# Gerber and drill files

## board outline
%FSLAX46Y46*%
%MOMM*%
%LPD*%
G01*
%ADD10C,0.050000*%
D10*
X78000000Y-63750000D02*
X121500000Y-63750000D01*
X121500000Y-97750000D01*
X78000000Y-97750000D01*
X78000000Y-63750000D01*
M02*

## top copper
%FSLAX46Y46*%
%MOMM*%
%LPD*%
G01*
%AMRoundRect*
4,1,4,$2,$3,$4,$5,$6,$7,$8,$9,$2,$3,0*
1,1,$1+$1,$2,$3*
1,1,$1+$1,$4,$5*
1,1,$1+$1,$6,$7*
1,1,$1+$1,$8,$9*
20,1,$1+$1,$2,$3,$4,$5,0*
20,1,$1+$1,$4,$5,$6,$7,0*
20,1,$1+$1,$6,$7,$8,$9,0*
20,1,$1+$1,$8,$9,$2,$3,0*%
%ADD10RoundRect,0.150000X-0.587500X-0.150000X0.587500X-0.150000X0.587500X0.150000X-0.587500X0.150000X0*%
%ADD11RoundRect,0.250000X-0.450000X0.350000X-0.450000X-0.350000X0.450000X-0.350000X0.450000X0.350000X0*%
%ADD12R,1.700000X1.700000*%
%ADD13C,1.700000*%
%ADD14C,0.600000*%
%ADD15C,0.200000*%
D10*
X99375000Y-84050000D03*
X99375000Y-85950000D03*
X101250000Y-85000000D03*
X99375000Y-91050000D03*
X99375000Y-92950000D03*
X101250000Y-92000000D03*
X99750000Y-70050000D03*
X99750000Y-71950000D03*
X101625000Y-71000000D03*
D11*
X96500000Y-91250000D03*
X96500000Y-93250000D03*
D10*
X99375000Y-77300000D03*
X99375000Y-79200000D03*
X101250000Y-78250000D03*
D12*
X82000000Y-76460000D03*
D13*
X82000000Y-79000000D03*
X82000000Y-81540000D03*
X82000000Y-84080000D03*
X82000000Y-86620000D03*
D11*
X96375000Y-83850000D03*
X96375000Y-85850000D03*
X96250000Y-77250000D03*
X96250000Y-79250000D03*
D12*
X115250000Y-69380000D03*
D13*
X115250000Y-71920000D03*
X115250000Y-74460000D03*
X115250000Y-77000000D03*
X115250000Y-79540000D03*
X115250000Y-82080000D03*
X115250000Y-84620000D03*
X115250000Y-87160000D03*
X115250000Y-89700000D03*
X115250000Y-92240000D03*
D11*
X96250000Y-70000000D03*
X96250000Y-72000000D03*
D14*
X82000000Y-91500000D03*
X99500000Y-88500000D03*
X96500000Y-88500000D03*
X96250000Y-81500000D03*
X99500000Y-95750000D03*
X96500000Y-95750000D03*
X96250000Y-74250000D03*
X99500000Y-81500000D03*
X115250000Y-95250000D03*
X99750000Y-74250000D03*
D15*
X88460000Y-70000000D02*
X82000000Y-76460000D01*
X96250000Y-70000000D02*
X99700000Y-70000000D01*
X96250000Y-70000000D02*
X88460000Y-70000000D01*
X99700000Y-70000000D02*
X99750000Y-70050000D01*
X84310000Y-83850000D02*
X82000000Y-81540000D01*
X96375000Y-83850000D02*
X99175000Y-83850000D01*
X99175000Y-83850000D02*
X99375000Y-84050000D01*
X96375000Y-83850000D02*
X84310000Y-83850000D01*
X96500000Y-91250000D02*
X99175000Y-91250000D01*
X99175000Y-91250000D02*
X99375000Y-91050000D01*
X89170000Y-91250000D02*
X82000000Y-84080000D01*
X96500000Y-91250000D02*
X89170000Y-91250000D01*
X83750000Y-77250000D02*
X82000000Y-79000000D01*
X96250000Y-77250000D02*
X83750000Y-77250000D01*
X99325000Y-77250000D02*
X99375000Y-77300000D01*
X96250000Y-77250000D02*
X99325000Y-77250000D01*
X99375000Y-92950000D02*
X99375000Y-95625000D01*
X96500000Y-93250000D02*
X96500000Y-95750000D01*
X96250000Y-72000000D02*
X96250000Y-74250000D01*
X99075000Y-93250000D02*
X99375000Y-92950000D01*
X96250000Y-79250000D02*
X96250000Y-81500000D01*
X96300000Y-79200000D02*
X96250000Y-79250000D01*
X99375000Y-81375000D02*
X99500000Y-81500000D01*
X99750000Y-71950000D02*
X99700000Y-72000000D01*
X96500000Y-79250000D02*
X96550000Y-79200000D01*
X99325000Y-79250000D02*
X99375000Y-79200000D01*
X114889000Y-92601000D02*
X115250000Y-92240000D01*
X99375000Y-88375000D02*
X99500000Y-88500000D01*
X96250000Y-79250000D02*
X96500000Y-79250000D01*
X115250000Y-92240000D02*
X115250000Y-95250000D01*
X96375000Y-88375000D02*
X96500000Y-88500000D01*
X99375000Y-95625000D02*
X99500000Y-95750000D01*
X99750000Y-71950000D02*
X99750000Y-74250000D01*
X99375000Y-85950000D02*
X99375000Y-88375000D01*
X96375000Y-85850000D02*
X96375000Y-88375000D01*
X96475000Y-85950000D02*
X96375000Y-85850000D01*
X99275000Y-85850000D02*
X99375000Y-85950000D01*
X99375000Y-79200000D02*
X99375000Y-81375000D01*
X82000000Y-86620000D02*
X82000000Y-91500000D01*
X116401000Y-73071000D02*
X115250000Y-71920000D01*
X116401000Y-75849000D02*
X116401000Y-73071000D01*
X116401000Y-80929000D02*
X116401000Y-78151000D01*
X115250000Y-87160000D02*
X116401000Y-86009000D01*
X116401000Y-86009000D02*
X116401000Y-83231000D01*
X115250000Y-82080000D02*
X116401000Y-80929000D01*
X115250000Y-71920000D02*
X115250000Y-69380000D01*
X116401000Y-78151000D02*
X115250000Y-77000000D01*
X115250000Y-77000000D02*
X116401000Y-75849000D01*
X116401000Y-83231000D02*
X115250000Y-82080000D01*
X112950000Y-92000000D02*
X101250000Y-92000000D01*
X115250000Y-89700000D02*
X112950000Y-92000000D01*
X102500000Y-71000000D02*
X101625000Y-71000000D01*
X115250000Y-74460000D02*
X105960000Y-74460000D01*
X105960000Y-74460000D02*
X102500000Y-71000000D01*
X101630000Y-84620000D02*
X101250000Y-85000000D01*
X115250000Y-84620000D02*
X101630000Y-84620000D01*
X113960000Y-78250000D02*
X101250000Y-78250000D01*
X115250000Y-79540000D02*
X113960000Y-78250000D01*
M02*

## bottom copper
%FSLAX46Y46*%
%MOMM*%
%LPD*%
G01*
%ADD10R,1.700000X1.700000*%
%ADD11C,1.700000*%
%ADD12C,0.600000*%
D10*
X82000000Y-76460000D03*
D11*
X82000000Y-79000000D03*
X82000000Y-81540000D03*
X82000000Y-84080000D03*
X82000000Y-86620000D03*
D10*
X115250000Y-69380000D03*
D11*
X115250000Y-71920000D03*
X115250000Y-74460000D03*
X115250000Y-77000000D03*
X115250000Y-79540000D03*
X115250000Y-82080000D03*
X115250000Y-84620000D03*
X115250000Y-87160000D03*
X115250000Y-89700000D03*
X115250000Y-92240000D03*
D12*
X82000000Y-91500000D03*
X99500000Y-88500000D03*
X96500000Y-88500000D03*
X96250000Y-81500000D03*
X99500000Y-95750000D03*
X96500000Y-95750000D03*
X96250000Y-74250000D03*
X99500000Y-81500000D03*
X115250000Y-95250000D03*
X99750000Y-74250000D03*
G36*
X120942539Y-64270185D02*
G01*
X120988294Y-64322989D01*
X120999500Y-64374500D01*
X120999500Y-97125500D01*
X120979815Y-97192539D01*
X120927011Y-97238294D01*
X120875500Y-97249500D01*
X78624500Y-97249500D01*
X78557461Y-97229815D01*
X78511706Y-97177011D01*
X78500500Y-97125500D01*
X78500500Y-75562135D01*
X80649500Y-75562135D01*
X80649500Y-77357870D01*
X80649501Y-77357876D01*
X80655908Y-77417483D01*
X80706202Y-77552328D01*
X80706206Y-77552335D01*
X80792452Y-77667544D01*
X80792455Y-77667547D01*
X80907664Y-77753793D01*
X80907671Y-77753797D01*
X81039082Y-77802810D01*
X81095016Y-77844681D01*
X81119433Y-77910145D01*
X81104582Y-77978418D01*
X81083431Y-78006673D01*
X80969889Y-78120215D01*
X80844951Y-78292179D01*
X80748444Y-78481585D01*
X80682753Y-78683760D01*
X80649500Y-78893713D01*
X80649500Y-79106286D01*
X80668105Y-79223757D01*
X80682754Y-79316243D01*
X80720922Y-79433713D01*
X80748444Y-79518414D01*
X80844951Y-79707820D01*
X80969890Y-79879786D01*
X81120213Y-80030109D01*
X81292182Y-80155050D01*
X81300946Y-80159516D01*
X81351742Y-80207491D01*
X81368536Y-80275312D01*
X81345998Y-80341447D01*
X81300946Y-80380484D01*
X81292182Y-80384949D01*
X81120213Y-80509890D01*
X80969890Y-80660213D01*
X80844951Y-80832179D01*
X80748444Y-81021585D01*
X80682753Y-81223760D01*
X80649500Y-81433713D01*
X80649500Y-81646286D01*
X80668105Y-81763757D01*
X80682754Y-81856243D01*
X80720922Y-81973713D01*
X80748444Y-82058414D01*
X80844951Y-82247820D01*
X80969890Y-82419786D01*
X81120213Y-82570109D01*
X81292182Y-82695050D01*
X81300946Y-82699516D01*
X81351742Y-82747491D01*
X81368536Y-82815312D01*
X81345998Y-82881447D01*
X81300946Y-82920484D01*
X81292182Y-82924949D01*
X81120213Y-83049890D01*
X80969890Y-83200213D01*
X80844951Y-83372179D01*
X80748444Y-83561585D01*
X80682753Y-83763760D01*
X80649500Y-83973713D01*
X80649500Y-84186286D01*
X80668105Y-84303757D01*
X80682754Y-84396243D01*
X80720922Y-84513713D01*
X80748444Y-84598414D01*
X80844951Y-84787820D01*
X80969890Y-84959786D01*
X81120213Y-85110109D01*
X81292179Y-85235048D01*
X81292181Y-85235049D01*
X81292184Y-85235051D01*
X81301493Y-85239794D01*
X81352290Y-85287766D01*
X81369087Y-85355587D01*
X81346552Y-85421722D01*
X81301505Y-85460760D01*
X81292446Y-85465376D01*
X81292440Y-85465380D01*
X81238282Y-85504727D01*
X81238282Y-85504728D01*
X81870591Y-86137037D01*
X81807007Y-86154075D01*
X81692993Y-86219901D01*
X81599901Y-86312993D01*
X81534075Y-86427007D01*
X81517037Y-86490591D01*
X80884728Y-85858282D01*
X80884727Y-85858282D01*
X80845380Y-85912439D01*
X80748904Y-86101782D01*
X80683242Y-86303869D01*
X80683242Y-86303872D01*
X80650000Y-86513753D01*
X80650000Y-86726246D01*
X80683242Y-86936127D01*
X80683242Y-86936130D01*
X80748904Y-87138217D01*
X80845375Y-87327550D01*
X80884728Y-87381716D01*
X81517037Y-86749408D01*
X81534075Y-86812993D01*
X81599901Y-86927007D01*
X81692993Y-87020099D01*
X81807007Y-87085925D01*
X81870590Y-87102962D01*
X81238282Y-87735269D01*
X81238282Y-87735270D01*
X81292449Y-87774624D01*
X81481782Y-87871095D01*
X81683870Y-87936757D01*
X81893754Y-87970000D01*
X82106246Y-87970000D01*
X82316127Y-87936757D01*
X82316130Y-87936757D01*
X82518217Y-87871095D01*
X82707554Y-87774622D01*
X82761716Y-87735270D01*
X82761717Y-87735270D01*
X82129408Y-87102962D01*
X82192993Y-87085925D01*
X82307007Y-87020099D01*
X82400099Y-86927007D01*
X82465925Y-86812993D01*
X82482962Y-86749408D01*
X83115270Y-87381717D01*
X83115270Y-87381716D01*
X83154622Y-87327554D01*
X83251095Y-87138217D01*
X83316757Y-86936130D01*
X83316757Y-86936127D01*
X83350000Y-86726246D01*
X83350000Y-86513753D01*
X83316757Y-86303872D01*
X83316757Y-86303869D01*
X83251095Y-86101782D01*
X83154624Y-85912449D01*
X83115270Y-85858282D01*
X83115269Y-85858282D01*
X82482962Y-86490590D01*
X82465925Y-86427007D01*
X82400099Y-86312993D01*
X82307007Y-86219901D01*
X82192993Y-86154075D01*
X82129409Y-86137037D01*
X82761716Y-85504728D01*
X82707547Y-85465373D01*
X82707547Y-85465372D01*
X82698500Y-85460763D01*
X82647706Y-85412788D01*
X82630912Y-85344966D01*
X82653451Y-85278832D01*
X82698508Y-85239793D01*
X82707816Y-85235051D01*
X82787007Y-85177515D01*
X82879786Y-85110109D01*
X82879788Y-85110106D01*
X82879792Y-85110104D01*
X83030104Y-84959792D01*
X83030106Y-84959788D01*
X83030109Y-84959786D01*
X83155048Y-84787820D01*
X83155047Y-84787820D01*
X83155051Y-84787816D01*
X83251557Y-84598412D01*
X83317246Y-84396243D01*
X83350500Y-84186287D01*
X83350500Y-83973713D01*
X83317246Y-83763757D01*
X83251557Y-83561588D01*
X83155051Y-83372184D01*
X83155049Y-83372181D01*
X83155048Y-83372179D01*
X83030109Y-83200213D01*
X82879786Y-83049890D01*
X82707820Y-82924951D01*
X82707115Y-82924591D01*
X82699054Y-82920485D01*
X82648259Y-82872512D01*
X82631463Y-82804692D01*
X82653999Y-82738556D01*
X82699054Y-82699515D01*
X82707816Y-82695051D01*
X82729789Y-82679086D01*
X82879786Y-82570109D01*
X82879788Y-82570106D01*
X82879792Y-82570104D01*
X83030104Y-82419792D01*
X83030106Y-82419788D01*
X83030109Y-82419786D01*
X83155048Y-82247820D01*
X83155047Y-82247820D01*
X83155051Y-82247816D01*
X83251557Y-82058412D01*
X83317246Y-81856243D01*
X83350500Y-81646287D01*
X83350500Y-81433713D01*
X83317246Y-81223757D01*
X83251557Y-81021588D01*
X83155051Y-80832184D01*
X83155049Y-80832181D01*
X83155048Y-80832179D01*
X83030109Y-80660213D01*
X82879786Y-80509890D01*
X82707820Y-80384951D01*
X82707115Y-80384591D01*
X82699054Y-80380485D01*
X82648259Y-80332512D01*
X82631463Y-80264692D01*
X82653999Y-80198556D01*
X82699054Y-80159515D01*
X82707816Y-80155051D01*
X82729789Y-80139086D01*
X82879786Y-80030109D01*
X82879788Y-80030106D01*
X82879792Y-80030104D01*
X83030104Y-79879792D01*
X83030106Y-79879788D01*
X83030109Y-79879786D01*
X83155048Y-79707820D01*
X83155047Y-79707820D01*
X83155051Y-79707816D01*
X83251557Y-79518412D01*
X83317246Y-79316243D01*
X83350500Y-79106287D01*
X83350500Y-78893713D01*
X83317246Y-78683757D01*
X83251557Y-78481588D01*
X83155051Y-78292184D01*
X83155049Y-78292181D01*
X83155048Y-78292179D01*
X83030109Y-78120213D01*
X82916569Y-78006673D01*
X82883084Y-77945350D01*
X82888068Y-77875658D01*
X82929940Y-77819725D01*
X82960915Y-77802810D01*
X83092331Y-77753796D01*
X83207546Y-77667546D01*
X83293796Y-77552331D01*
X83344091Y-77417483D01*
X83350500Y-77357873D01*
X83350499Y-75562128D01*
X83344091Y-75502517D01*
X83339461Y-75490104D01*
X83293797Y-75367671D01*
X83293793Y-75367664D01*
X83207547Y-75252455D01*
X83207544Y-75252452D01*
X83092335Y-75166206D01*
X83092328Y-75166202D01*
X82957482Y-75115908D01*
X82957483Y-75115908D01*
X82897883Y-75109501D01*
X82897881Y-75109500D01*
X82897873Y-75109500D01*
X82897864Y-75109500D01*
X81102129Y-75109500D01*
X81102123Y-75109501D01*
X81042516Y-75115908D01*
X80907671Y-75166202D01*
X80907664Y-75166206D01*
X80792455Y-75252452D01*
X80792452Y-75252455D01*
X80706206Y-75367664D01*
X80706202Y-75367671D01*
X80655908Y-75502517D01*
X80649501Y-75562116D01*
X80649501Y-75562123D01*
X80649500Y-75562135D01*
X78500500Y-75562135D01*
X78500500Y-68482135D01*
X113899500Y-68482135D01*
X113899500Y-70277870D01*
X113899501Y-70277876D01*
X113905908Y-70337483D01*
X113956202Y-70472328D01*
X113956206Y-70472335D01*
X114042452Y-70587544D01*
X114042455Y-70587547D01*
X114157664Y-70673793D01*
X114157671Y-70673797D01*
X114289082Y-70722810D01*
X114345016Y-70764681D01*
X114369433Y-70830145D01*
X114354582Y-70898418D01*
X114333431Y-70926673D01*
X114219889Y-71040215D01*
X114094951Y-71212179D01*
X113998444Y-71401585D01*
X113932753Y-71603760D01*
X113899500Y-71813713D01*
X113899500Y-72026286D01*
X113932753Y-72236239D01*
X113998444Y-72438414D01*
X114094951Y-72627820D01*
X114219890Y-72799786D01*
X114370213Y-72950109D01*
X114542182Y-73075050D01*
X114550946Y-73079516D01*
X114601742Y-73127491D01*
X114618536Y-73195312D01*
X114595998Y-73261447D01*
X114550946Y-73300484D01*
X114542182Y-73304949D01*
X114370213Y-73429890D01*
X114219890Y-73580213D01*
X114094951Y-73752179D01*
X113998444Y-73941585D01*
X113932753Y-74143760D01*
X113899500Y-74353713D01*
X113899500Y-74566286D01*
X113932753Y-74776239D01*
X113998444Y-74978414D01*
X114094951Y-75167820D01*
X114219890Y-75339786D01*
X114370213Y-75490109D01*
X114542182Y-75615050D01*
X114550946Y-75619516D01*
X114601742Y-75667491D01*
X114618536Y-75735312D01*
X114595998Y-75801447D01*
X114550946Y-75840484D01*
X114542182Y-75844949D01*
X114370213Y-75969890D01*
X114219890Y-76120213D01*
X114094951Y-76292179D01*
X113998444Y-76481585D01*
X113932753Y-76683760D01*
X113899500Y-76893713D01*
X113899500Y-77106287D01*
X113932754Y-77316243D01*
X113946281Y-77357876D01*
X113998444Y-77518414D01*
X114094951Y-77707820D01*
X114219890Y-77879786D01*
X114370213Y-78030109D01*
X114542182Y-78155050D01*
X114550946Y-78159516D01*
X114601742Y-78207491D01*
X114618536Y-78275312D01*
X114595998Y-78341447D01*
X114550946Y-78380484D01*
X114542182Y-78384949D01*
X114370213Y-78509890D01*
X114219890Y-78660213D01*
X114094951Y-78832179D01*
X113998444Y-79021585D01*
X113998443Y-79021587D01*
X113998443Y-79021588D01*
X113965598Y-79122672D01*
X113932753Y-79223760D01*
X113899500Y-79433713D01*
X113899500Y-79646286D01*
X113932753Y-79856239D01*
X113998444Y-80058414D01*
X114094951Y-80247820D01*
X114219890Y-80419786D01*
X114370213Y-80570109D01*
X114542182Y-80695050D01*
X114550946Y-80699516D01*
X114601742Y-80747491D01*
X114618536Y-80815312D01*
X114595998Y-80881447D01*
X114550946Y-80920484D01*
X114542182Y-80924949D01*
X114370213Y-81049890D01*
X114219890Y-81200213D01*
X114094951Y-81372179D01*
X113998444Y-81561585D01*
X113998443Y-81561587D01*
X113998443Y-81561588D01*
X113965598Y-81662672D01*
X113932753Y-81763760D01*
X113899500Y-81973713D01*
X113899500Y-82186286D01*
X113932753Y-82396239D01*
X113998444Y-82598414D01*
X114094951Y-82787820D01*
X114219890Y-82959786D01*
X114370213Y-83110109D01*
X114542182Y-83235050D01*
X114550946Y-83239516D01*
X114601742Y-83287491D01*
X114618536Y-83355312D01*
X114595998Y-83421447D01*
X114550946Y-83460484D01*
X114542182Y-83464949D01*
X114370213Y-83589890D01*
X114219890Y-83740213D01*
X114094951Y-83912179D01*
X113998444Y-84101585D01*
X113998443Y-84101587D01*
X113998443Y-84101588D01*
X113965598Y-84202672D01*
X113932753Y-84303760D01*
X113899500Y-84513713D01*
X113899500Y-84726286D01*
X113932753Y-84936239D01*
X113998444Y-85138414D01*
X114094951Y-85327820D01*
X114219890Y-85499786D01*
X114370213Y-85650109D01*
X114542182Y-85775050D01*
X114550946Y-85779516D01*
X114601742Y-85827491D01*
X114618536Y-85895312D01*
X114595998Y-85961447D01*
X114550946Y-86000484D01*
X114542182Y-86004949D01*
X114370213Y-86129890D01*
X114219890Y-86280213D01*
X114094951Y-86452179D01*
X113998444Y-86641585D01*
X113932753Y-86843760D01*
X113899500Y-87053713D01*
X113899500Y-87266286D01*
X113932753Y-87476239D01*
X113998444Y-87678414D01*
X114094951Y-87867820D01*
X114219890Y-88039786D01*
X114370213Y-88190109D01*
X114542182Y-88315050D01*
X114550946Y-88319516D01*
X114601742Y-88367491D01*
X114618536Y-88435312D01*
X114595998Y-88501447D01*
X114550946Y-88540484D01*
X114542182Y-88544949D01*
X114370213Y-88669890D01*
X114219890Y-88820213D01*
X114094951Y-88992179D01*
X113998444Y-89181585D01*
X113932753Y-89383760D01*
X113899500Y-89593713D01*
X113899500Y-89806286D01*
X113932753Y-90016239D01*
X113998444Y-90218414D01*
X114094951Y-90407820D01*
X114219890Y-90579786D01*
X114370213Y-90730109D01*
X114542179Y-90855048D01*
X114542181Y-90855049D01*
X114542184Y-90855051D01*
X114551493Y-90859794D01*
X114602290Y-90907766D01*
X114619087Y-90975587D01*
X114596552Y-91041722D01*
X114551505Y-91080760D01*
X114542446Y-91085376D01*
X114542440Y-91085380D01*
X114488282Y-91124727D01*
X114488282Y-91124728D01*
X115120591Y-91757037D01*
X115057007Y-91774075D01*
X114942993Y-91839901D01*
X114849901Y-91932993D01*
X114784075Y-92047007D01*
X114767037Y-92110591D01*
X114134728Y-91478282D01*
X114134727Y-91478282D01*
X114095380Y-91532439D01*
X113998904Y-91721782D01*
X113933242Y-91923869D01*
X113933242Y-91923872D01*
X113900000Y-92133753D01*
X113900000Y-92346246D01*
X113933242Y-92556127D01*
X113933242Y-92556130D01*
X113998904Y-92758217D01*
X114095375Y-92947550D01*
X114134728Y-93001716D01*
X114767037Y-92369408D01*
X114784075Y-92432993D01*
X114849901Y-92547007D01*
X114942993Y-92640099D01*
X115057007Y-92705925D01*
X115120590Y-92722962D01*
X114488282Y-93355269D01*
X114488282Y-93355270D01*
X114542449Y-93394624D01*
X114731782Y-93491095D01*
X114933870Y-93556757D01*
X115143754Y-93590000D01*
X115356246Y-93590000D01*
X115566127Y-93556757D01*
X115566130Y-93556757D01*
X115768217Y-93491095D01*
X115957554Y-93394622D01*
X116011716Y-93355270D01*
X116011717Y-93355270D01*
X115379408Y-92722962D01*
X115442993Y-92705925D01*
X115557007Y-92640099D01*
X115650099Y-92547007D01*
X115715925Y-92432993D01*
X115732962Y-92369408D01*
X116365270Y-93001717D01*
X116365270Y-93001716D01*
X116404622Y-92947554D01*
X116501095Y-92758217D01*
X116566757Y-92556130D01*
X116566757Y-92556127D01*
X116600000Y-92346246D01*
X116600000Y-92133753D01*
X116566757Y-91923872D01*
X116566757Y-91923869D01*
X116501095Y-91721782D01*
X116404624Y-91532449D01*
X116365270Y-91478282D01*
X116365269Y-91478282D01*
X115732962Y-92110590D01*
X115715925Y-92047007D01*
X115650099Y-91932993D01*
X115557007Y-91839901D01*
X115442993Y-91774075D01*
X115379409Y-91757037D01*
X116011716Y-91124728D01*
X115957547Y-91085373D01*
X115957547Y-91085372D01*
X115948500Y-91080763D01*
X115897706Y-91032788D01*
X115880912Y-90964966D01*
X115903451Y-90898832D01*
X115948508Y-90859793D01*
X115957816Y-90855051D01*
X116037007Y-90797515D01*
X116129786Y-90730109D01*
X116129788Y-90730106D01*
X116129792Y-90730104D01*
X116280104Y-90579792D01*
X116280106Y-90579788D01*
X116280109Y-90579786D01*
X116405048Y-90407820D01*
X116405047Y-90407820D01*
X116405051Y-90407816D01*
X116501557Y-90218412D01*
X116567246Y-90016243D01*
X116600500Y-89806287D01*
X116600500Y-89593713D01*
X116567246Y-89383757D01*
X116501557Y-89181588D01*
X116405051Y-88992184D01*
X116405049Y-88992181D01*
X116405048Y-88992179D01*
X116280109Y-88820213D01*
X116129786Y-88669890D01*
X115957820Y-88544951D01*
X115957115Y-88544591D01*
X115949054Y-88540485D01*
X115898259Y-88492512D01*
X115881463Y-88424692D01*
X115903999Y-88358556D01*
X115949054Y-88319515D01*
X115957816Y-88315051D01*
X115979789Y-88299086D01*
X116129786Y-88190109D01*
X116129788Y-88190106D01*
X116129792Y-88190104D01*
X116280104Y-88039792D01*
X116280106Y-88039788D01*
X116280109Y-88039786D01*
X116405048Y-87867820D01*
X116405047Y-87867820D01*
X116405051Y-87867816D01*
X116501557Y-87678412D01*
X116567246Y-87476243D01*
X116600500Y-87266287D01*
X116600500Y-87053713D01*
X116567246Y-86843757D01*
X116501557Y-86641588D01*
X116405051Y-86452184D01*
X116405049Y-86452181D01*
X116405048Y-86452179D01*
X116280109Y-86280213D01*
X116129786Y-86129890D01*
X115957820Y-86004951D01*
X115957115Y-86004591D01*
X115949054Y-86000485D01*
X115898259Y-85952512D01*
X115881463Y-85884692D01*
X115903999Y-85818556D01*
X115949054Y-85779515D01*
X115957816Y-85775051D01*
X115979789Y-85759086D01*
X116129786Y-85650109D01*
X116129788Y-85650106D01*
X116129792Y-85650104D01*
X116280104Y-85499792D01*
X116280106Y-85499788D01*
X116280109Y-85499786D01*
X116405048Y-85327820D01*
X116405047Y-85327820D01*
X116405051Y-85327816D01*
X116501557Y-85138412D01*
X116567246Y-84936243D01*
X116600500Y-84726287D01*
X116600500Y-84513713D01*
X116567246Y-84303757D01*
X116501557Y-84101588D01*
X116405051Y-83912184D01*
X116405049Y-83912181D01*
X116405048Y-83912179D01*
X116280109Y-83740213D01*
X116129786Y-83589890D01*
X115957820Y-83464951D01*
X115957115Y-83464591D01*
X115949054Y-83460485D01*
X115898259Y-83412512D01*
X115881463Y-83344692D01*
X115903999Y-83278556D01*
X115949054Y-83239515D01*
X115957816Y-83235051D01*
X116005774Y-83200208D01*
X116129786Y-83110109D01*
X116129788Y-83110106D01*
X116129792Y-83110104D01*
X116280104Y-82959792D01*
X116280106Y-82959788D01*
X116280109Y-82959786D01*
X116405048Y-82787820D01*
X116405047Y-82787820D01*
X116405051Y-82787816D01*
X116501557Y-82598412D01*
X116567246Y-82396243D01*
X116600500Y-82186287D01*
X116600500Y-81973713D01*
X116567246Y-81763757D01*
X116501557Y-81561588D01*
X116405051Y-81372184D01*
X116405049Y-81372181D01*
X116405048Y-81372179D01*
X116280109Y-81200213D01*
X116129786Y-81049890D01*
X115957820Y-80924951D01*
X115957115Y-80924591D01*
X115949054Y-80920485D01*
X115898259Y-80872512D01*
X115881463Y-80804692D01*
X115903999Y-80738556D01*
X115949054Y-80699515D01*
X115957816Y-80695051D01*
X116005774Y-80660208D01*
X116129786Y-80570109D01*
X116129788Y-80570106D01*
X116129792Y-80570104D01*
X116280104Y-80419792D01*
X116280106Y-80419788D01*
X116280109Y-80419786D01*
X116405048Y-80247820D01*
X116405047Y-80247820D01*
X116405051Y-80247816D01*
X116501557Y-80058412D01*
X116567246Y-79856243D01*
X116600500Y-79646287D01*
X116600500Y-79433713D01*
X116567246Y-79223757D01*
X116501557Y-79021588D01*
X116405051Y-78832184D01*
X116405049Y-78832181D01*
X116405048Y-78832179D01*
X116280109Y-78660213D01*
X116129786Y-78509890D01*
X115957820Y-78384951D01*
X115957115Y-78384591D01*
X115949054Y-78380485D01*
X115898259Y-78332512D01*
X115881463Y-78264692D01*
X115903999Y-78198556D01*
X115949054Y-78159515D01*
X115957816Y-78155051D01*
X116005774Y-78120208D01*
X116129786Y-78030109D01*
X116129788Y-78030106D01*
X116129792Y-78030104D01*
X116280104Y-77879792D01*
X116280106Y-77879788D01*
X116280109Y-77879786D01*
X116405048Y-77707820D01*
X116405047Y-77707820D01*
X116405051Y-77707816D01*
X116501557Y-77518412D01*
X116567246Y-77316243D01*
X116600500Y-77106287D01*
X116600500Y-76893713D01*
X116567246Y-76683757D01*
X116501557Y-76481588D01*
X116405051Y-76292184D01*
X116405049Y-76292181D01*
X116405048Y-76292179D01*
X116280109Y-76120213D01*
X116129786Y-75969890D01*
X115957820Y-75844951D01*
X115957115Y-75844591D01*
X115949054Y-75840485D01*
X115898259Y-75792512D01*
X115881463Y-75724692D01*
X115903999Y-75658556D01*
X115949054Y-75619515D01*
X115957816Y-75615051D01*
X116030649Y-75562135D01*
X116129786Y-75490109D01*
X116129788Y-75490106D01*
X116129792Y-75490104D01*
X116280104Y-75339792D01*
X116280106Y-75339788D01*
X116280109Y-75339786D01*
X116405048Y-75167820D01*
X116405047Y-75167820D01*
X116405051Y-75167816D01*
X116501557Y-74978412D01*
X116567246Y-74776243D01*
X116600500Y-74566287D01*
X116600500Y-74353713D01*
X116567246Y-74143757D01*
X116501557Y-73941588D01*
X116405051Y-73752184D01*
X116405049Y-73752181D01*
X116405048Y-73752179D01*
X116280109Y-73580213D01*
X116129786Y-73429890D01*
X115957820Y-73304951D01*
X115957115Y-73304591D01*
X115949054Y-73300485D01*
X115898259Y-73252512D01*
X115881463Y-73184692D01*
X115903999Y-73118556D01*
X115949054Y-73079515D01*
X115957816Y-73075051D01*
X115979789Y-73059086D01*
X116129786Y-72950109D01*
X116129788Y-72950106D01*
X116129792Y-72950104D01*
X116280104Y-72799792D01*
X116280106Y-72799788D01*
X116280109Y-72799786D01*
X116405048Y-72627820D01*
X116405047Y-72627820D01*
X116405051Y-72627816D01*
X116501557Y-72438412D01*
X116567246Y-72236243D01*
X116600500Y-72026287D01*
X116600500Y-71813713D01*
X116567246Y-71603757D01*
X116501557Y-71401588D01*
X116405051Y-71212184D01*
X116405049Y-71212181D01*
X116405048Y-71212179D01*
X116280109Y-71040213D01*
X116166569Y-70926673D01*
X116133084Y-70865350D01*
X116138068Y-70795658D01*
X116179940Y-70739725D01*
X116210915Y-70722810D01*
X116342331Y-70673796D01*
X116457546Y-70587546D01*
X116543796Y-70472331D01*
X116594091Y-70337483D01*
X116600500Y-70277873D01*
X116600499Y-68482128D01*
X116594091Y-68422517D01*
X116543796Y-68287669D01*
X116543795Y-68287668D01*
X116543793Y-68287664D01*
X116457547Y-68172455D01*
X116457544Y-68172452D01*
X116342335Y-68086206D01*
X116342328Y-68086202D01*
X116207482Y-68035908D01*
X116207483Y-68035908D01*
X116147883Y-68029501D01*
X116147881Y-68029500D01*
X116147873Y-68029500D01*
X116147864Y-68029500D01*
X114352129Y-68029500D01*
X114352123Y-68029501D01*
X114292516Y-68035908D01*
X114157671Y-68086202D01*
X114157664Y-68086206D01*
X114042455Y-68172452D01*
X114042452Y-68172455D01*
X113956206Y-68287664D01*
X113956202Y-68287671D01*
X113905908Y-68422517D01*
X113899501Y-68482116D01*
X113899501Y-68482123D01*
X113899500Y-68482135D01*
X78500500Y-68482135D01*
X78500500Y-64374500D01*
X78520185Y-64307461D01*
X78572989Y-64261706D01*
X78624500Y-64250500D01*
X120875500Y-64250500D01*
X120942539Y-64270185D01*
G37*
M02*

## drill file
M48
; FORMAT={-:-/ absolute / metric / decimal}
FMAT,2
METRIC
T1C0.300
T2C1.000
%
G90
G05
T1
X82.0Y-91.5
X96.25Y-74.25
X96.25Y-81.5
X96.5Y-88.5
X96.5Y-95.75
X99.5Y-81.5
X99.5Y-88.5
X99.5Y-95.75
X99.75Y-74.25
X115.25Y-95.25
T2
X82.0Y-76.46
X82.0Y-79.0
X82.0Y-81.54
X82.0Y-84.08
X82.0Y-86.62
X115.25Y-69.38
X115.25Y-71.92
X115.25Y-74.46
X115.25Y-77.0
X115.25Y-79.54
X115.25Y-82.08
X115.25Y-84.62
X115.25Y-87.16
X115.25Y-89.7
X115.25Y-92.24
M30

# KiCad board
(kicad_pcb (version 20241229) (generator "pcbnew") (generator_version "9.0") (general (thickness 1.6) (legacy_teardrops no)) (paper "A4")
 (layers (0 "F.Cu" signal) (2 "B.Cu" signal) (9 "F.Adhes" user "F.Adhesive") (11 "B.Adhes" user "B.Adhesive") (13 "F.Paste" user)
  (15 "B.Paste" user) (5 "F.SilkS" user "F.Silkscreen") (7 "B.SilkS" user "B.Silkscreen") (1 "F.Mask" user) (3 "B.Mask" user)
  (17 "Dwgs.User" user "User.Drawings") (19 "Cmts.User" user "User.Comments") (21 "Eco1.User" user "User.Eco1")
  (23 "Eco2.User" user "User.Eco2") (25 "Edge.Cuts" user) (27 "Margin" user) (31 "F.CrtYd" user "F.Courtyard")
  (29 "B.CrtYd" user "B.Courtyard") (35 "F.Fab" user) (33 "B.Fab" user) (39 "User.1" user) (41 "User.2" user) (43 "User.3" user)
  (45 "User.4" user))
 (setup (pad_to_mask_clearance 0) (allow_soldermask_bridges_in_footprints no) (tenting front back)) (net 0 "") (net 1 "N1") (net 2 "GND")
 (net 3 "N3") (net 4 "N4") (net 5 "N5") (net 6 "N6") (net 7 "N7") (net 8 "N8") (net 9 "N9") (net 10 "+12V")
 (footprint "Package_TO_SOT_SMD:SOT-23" (layer "F.Cu") (at 100.3125 85)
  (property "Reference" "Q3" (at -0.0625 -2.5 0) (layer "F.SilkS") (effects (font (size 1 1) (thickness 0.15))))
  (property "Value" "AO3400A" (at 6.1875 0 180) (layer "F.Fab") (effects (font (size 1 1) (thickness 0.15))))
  (pad "1" smd roundrect (at -0.9375 -0.95) (size 1.475 0.6) (layers "F.Cu" "F.Mask" "F.Paste") (roundrect_rratio 0.25) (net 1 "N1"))
  (pad "2" smd roundrect (at -0.9375 0.95) (size 1.475 0.6) (layers "F.Cu" "F.Mask" "F.Paste") (roundrect_rratio 0.25) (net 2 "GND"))
  (pad "3" smd roundrect (at 0.9375 0) (size 1.475 0.6) (layers "F.Cu" "F.Mask" "F.Paste") (roundrect_rratio 0.25) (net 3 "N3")))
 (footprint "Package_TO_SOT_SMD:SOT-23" (layer "F.Cu") (at 100.3125 92)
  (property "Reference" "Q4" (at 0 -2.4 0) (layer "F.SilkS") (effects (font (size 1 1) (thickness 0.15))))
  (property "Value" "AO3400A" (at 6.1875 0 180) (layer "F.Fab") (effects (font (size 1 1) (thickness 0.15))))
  (pad "1" smd roundrect (at -0.9375 -0.95) (size 1.475 0.6) (layers "F.Cu" "F.Mask" "F.Paste") (roundrect_rratio 0.25) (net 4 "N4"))
  (pad "2" smd roundrect (at -0.9375 0.95) (size 1.475 0.6) (layers "F.Cu" "F.Mask" "F.Paste") (roundrect_rratio 0.25) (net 2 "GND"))
  (pad "3" smd roundrect (at 0.9375 0) (size 1.475 0.6) (layers "F.Cu" "F.Mask" "F.Paste") (roundrect_rratio 0.25) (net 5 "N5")))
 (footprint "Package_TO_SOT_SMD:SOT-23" (layer "F.Cu") (at 100.6875 71)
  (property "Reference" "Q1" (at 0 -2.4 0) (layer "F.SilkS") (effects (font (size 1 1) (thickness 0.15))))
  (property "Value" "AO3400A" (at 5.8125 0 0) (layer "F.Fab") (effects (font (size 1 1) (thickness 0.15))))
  (pad "1" smd roundrect (at -0.9375 -0.95) (size 1.475 0.6) (layers "F.Cu" "F.Mask" "F.Paste") (roundrect_rratio 0.25) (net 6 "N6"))
  (pad "2" smd roundrect (at -0.9375 0.95) (size 1.475 0.6) (layers "F.Cu" "F.Mask" "F.Paste") (roundrect_rratio 0.25) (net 2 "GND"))
  (pad "3" smd roundrect (at 0.9375 0) (size 1.475 0.6) (layers "F.Cu" "F.Mask" "F.Paste") (roundrect_rratio 0.25) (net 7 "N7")))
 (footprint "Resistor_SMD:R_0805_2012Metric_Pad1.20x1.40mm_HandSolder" (layer "F.Cu") (at 96.5 92.25 -90)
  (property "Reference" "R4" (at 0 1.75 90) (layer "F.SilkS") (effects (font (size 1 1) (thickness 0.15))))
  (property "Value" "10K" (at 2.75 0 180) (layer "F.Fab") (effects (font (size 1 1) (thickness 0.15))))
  (pad "1" smd roundrect (at -1 0 270) (size 1.2 1.4) (layers "F.Cu" "F.Mask" "F.Paste") (roundrect_rratio 0.208333) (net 4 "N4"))
  (pad "2" smd roundrect (at 1 0 270) (size 1.2 1.4) (layers "F.Cu" "F.Mask" "F.Paste") (roundrect_rratio 0.208333) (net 2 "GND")))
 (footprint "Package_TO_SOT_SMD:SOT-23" (layer "F.Cu") (at 100.3125 78.25)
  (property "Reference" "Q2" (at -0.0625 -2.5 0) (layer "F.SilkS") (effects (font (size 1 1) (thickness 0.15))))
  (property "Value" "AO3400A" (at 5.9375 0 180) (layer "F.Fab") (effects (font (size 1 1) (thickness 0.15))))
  (pad "1" smd roundrect (at -0.9375 -0.95) (size 1.475 0.6) (layers "F.Cu" "F.Mask" "F.Paste") (roundrect_rratio 0.25) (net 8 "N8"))
  (pad "2" smd roundrect (at -0.9375 0.95) (size 1.475 0.6) (layers "F.Cu" "F.Mask" "F.Paste") (roundrect_rratio 0.25) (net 2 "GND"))
  (pad "3" smd roundrect (at 0.9375 0) (size 1.475 0.6) (layers "F.Cu" "F.Mask" "F.Paste") (roundrect_rratio 0.25) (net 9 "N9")))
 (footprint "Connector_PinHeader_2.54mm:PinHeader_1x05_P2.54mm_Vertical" (layer "F.Cu") (at 82 76.46)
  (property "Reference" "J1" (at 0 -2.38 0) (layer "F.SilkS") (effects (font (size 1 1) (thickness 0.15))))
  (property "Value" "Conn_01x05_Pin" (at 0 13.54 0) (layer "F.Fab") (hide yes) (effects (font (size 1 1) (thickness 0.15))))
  (pad "1" thru_hole rect (at 0 0) (size 1.7 1.7) (drill 1) (layers "*.Cu" "*.Mask") (remove_unused_layers no) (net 6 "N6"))
  (pad "2" thru_hole circle (at 0 2.54) (size 1.7 1.7) (drill 1) (layers "*.Cu" "*.Mask") (remove_unused_layers no) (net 8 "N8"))
  (pad "3" thru_hole circle (at 0 5.08) (size 1.7 1.7) (drill 1) (layers "*.Cu" "*.Mask") (remove_unused_layers no) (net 1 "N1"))
  (pad "4" thru_hole circle (at 0 7.62) (size 1.7 1.7) (drill 1) (layers "*.Cu" "*.Mask") (remove_unused_layers no) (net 4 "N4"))
  (pad "5" thru_hole circle (at 0 10.16) (size 1.7 1.7) (drill 1) (layers "*.Cu" "*.Mask") (remove_unused_layers no) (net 2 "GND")))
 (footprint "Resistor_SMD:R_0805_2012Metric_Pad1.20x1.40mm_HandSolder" (layer "F.Cu") (at 96.375 84.85 -90)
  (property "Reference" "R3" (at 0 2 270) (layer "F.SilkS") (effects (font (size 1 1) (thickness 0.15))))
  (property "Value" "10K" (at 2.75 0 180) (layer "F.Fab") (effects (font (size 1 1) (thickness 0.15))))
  (pad "1" smd roundrect (at -1 0 270) (size 1.2 1.4) (layers "F.Cu" "F.Mask" "F.Paste") (roundrect_rratio 0.208333) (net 1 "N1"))
  (pad "2" smd roundrect (at 1 0 270) (size 1.2 1.4) (layers "F.Cu" "F.Mask" "F.Paste") (roundrect_rratio 0.208333) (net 2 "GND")))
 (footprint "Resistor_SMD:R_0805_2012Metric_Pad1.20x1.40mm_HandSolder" (layer "F.Cu") (at 96.25 78.25 -90)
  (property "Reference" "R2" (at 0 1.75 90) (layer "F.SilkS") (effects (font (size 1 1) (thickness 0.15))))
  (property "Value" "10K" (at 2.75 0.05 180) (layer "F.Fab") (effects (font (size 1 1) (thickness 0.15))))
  (pad "1" smd roundrect (at -1 0 270) (size 1.2 1.4) (layers "F.Cu" "F.Mask" "F.Paste") (roundrect_rratio 0.208333) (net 8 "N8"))
  (pad "2" smd roundrect (at 1 0 270) (size 1.2 1.4) (layers "F.Cu" "F.Mask" "F.Paste") (roundrect_rratio 0.208333) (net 2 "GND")))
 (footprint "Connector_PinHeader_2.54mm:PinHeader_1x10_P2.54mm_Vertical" (layer "F.Cu") (at 115.25 69.38)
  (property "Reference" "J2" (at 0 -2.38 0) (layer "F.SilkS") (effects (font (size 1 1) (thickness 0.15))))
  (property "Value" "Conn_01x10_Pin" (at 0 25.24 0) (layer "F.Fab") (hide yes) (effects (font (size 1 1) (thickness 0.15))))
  (pad "1" thru_hole rect (at 0 0) (size 1.7 1.7) (drill 1) (layers "*.Cu" "*.Mask") (remove_unused_layers no) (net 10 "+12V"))
  (pad "2" thru_hole circle (at 0 2.54) (size 1.7 1.7) (drill 1) (layers "*.Cu" "*.Mask") (remove_unused_layers no) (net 10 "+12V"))
  (pad "3" thru_hole circle (at 0 5.08) (size 1.7 1.7) (drill 1) (layers "*.Cu" "*.Mask") (remove_unused_layers no) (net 7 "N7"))
  (pad "4" thru_hole circle (at 0 7.62) (size 1.7 1.7) (drill 1) (layers "*.Cu" "*.Mask") (remove_unused_layers no) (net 10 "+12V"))
  (pad "5" thru_hole circle (at 0 10.16) (size 1.7 1.7) (drill 1) (layers "*.Cu" "*.Mask") (remove_unused_layers no) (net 9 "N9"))
  (pad "6" thru_hole circle (at 0 12.7) (size 1.7 1.7) (drill 1) (layers "*.Cu" "*.Mask") (remove_unused_layers no) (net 10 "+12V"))
  (pad "7" thru_hole circle (at 0 15.24) (size 1.7 1.7) (drill 1) (layers "*.Cu" "*.Mask") (remove_unused_layers no) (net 3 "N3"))
  (pad "8" thru_hole circle (at 0 17.78) (size 1.7 1.7) (drill 1) (layers "*.Cu" "*.Mask") (remove_unused_layers no) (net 10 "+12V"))
  (pad "9" thru_hole circle (at 0 20.32) (size 1.7 1.7) (drill 1) (layers "*.Cu" "*.Mask") (remove_unused_layers no) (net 5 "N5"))
  (pad "10" thru_hole circle (at 0 22.86) (size 1.7 1.7) (drill 1) (layers "*.Cu" "*.Mask") (remove_unused_layers no) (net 2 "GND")))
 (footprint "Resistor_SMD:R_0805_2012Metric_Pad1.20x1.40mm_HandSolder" (layer "F.Cu") (at 96.25 71 -90)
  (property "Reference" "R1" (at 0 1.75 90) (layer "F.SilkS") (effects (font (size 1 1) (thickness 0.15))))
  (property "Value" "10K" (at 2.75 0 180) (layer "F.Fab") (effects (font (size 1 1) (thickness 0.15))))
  (pad "1" smd roundrect (at -1 0 270) (size 1.2 1.4) (layers "F.Cu" "F.Mask" "F.Paste") (roundrect_rratio 0.208333) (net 6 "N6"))
  (pad "2" smd roundrect (at 1 0 270) (size 1.2 1.4) (layers "F.Cu" "F.Mask" "F.Paste") (roundrect_rratio 0.208333) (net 2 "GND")))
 (gr_rect (start 78 63.75) (end 121.5 97.75) (stroke (width 0.05) (type solid)) (fill no) (layer "Edge.Cuts"))
 (segment (start 88.46 70) (end 82 76.46) (width 0.2) (layer "F.Cu") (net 6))
 (segment (start 96.25 70) (end 99.7 70) (width 0.2) (layer "F.Cu") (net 6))
 (segment (start 96.25 70) (end 88.46 70) (width 0.2) (layer "F.Cu") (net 6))
 (segment (start 99.7 70) (end 99.75 70.05) (width 0.2) (layer "F.Cu") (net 6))
 (segment (start 84.31 83.85) (end 82 81.54) (width 0.2) (layer "F.Cu") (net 1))
 (segment (start 96.375 83.85) (end 99.175 83.85) (width 0.2) (layer "F.Cu") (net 1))
 (segment (start 99.175 83.85) (end 99.375 84.05) (width 0.2) (layer "F.Cu") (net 1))
 (segment (start 96.375 83.85) (end 84.31 83.85) (width 0.2) (layer "F.Cu") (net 1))
 (segment (start 96.5 91.25) (end 99.175 91.25) (width 0.2) (layer "F.Cu") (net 4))
 (segment (start 99.175 91.25) (end 99.375 91.05) (width 0.2) (layer "F.Cu") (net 4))
 (segment (start 89.17 91.25) (end 82 84.08) (width 0.2) (layer "F.Cu") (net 4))
 (segment (start 96.5 91.25) (end 89.17 91.25) (width 0.2) (layer "F.Cu") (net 4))
 (segment (start 83.75 77.25) (end 82 79) (width 0.2) (layer "F.Cu") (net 8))
 (segment (start 96.25 77.25) (end 83.75 77.25) (width 0.2) (layer "F.Cu") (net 8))
 (segment (start 99.325 77.25) (end 99.375 77.3) (width 0.2) (layer "F.Cu") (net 8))
 (segment (start 96.25 77.25) (end 99.325 77.25) (width 0.2) (layer "F.Cu") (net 8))
 (segment (start 99.375 92.95) (end 99.375 95.625) (width 0.2) (layer "F.Cu") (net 2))
 (segment (start 96.5 93.25) (end 96.5 95.75) (width 0.2) (layer "F.Cu") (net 2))
 (segment (start 96.25 72) (end 96.25 74.25) (width 0.2) (layer "F.Cu") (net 2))
 (segment (start 99.075 93.25) (end 99.375 92.95) (width 0.2) (layer "F.Cu") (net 2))
 (segment (start 96.25 79.25) (end 96.25 81.5) (width 0.2) (layer "F.Cu") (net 2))
 (segment (start 96.3 79.2) (end 96.25 79.25) (width 0.2) (layer "F.Cu") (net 2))
 (segment (start 99.375 81.375) (end 99.5 81.5) (width 0.2) (layer "F.Cu") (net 2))
 (segment (start 99.75 71.95) (end 99.7 72) (width 0.2) (layer "F.Cu") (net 2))
 (segment (start 96.5 79.25) (end 96.55 79.2) (width 0.2) (layer "F.Cu") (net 2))
 (segment (start 99.325 79.25) (end 99.375 79.2) (width 0.2) (layer "F.Cu") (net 2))
 (segment (start 114.889 92.601) (end 115.25 92.24) (width 0.2) (layer "F.Cu") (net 2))
 (segment (start 99.375 88.375) (end 99.5 88.5) (width 0.2) (layer "F.Cu") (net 2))
 (segment (start 96.25 79.25) (end 96.5 79.25) (width 0.2) (layer "F.Cu") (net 2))
 (segment (start 115.25 92.24) (end 115.25 95.25) (width 0.2) (layer "F.Cu") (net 2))
 (segment (start 96.375 88.375) (end 96.5 88.5) (width 0.2) (layer "F.Cu") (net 2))
 (segment (start 99.375 95.625) (end 99.5 95.75) (width 0.2) (layer "F.Cu") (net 2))
 (segment (start 99.75 71.95) (end 99.75 74.25) (width 0.2) (layer "F.Cu") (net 2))
 (segment (start 99.375 85.95) (end 99.375 88.375) (width 0.2) (layer "F.Cu") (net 2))
 (segment (start 96.375 85.85) (end 96.375 88.375) (width 0.2) (layer "F.Cu") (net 2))
 (segment (start 96.475 85.95) (end 96.375 85.85) (width 0.2) (layer "F.Cu") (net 2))
 (segment (start 99.275 85.85) (end 99.375 85.95) (width 0.2) (layer "F.Cu") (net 2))
 (segment (start 99.375 79.2) (end 99.375 81.375) (width 0.2) (layer "F.Cu") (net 2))
 (segment (start 82 86.62) (end 82 91.5) (width 0.2) (layer "F.Cu") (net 2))
 (via (at 82 91.5) (size 0.6) (drill 0.3) (layers "F.Cu" "B.Cu") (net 2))
 (via (at 99.5 88.5) (size 0.6) (drill 0.3) (layers "F.Cu" "B.Cu") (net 2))
 (via (at 96.5 88.5) (size 0.6) (drill 0.3) (layers "F.Cu" "B.Cu") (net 2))
 (via (at 96.25 81.5) (size 0.6) (drill 0.3) (layers "F.Cu" "B.Cu") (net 2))
 (via (at 99.5 95.75) (size 0.6) (drill 0.3) (layers "F.Cu" "B.Cu") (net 2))
 (via (at 96.5 95.75) (size 0.6) (drill 0.3) (layers "F.Cu" "B.Cu") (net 2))
 (via (at 96.25 74.25) (size 0.6) (drill 0.3) (layers "F.Cu" "B.Cu") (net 2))
 (via (at 99.5 81.5) (size 0.6) (drill 0.3) (layers "F.Cu" "B.Cu") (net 2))
 (via (at 115.25 95.25) (size 0.6) (drill 0.3) (layers "F.Cu" "B.Cu") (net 2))
 (via (at 99.75 74.25) (size 0.6) (drill 0.3) (layers "F.Cu" "B.Cu") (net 2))
 (segment (start 116.401 73.071) (end 115.25 71.92) (width 0.2) (layer "F.Cu") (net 10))
 (segment (start 116.401 75.849) (end 116.401 73.071) (width 0.2) (layer "F.Cu") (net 10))
 (segment (start 116.401 80.929) (end 116.401 78.151) (width 0.2) (layer "F.Cu") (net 10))
 (segment (start 115.25 87.16) (end 116.401 86.009) (width 0.2) (layer "F.Cu") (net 10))
 (segment (start 116.401 86.009) (end 116.401 83.231) (width 0.2) (layer "F.Cu") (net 10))
 (segment (start 115.25 82.08) (end 116.401 80.929) (width 0.2) (layer "F.Cu") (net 10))
 (segment (start 115.25 71.92) (end 115.25 69.38) (width 0.2) (layer "F.Cu") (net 10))
 (segment (start 116.401 78.151) (end 115.25 77) (width 0.2) (layer "F.Cu") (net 10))
 (segment (start 115.25 77) (end 116.401 75.849) (width 0.2) (layer "F.Cu") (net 10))
 (segment (start 116.401 83.231) (end 115.25 82.08) (width 0.2) (layer "F.Cu") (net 10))
 (segment (start 112.95 92) (end 101.25 92) (width 0.2) (layer "F.Cu") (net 5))
 (segment (start 115.25 89.7) (end 112.95 92) (width 0.2) (layer "F.Cu") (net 5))
 (segment (start 102.5 71) (end 101.625 71) (width 0.2) (layer "F.Cu") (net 7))
 (segment (start 115.25 74.46) (end 105.96 74.46) (width 0.2) (layer "F.Cu") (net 7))
 (segment (start 105.96 74.46) (end 102.5 71) (width 0.2) (layer "F.Cu") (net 7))
 (segment (start 101.63 84.62) (end 101.25 85) (width 0.2) (layer "F.Cu") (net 3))
 (segment (start 115.25 84.62) (end 101.63 84.62) (width 0.2) (layer "F.Cu") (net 3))
 (segment (start 113.96 78.25) (end 101.25 78.25) (width 0.2) (layer "F.Cu") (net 9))
 (segment (start 115.25 79.54) (end 113.96 78.25) (width 0.2) (layer "F.Cu") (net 9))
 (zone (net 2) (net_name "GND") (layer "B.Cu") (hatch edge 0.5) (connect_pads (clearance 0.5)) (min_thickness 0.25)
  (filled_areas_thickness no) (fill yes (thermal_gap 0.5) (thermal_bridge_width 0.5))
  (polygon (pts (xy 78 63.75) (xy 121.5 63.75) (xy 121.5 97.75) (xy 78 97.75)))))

